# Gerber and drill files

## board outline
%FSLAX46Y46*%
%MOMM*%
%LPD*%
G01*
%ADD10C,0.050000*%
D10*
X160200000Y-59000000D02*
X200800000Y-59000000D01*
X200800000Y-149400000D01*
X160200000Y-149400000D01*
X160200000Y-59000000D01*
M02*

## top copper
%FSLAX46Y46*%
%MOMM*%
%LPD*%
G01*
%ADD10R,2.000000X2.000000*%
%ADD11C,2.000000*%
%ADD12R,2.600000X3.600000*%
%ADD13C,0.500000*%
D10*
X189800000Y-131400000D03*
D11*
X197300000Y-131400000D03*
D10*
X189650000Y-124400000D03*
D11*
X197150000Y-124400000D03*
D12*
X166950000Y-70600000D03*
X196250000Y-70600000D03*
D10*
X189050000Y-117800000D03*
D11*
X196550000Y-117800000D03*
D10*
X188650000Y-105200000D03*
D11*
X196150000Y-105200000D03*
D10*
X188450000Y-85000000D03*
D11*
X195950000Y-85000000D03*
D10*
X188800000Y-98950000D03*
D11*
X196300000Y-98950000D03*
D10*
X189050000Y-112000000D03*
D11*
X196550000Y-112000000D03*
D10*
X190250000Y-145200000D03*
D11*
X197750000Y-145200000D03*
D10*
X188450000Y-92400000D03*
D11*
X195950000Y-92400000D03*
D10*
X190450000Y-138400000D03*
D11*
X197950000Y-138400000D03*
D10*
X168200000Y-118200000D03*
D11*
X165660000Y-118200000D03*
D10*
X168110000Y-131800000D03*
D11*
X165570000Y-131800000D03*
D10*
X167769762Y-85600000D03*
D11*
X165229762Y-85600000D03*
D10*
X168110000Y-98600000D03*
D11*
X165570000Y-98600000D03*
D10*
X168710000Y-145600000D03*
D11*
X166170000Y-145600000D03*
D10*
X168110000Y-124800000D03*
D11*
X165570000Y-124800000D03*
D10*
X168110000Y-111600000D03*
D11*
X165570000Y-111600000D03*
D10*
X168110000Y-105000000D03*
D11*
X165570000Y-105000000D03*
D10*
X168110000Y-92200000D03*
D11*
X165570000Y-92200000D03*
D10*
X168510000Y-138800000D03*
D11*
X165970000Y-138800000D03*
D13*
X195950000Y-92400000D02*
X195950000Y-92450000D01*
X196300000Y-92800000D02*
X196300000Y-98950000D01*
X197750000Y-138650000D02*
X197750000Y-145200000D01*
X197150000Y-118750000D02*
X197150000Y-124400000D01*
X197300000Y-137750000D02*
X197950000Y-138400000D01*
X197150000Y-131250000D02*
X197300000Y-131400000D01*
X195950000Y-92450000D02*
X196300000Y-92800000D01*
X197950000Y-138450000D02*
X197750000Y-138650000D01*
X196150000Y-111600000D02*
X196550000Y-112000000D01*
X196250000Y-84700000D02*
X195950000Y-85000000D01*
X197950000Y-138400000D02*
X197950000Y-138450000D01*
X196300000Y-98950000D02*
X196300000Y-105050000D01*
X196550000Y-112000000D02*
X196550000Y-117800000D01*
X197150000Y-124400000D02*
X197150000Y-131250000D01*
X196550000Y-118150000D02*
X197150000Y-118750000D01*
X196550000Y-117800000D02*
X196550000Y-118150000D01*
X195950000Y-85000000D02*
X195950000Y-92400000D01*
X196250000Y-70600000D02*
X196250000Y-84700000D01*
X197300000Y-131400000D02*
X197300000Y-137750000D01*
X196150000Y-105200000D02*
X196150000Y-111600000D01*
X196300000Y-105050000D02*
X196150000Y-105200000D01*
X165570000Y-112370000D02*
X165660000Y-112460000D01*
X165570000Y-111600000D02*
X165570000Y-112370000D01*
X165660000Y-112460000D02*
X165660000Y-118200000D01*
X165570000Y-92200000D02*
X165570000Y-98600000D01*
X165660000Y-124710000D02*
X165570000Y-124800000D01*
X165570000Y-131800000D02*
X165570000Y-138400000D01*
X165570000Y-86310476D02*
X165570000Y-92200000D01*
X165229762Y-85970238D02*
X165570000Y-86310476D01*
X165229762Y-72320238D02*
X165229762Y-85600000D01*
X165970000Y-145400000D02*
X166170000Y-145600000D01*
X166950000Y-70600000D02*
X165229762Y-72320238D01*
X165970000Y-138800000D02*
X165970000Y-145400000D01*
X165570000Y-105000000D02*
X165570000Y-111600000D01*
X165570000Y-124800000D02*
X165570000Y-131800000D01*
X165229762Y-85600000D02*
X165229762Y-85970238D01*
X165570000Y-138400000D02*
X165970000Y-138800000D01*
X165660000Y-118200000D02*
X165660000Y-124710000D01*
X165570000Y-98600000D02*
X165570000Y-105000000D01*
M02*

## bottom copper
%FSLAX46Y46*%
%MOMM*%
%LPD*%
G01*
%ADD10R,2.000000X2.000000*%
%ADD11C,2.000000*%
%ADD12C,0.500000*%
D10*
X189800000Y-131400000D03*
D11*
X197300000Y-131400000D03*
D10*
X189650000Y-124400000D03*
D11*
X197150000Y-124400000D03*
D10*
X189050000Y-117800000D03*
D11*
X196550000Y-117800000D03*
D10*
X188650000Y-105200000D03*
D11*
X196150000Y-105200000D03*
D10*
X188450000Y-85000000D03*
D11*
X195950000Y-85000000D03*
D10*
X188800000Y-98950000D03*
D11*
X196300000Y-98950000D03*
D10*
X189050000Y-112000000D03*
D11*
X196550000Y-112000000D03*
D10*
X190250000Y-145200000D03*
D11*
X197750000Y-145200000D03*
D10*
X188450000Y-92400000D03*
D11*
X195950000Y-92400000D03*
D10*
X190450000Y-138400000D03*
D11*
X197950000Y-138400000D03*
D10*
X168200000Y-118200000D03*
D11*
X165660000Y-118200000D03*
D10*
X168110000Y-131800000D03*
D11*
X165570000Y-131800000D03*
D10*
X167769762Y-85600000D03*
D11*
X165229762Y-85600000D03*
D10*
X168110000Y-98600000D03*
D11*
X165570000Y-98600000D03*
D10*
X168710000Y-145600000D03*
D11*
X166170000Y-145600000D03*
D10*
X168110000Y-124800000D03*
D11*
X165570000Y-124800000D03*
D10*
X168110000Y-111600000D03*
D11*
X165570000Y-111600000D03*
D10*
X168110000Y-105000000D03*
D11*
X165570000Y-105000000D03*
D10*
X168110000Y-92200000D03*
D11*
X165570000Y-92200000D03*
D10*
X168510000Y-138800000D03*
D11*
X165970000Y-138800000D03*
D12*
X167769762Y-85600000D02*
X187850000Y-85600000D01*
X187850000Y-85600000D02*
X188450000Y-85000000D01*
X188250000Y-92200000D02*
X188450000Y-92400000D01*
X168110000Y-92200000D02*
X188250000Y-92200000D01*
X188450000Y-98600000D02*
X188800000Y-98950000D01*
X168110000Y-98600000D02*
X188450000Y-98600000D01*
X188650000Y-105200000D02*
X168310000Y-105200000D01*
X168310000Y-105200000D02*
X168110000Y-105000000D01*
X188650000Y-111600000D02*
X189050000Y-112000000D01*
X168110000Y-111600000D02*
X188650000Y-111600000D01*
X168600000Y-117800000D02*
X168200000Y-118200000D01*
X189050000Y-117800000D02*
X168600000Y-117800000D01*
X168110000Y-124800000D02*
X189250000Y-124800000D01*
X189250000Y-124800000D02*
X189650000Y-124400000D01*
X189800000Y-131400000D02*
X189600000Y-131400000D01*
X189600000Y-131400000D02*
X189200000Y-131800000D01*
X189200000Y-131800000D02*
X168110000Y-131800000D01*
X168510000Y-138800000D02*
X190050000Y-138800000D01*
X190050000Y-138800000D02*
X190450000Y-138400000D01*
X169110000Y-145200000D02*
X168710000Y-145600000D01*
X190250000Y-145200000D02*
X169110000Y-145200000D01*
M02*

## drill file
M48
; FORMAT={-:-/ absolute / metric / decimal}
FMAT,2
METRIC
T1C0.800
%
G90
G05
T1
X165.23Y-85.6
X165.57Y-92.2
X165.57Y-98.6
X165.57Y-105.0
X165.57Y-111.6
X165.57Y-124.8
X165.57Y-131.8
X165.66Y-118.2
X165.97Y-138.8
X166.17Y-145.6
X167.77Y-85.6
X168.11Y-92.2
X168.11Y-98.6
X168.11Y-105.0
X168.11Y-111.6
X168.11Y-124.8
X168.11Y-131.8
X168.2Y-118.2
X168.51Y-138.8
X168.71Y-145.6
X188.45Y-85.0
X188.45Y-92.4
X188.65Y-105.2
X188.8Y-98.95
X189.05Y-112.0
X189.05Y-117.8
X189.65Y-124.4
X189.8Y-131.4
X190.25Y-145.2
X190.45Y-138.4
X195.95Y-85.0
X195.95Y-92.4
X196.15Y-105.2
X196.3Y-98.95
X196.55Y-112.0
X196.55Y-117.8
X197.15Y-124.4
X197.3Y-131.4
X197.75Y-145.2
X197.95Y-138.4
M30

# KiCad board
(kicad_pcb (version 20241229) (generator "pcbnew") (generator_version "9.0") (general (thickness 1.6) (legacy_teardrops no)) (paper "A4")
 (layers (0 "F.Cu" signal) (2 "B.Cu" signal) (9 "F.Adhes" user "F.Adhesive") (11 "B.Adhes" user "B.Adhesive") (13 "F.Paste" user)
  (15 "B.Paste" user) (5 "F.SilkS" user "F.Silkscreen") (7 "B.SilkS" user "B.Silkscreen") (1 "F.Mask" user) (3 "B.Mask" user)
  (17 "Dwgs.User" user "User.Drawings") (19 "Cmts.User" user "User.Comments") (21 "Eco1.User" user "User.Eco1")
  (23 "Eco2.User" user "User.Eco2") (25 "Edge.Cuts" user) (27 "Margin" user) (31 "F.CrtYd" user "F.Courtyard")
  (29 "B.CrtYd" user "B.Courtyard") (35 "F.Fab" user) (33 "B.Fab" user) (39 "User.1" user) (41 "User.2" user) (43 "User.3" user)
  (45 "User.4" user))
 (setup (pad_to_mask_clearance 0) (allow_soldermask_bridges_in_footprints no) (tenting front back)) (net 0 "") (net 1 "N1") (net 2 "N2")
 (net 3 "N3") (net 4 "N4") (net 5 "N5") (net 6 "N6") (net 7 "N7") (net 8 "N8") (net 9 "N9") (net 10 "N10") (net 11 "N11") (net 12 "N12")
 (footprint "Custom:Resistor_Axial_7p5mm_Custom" (layer "F.Cu") (at 189.8 131.4)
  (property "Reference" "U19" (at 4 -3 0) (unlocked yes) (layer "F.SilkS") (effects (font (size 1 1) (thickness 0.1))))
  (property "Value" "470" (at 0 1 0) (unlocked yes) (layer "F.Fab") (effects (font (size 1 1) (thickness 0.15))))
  (pad "1" thru_hole rect (at 0 0) (size 2 2) (drill 0.8) (layers "*.Cu" "*.Mask") (remove_unused_layers no) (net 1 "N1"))
  (pad "2" thru_hole circle (at 7.5 0) (size 2 2) (drill 0.8) (layers "*.Cu" "*.Mask") (remove_unused_layers no) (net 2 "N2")))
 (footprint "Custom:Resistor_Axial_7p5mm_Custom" (layer "F.Cu") (at 189.65 124.4)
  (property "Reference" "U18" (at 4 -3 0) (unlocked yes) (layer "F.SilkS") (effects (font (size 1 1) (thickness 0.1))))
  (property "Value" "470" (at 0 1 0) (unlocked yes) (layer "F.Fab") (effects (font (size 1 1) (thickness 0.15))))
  (pad "1" thru_hole rect (at 0 0) (size 2 2) (drill 0.8) (layers "*.Cu" "*.Mask") (remove_unused_layers no) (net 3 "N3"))
  (pad "2" thru_hole circle (at 7.5 0) (size 2 2) (drill 0.8) (layers "*.Cu" "*.Mask") (remove_unused_layers no) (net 2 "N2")))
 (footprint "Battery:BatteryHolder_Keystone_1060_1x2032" (layer "F.Cu") (at 181.6 70.6)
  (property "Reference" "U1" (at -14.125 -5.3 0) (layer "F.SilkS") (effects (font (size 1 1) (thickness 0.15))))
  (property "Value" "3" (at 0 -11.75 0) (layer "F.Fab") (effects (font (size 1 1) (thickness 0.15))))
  (pad "1" smd rect (at -14.65 0 180) (size 2.6 3.6) (layers "F.Cu" "F.Mask" "F.Paste") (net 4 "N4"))
  (pad "2" smd rect (at 14.65 0 180) (size 2.6 3.6) (layers "F.Cu" "F.Mask" "F.Paste") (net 2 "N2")))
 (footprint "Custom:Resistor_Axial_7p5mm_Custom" (layer "F.Cu") (at 189.05 117.8)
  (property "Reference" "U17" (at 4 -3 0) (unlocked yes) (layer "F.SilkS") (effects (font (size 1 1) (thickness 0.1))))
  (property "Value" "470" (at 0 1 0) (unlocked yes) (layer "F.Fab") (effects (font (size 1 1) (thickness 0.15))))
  (pad "1" thru_hole rect (at 0 0) (size 2 2) (drill 0.8) (layers "*.Cu" "*.Mask") (remove_unused_layers no) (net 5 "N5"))
  (pad "2" thru_hole circle (at 7.5 0) (size 2 2) (drill 0.8) (layers "*.Cu" "*.Mask") (remove_unused_layers no) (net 2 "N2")))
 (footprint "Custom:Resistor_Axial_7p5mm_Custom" (layer "F.Cu") (at 188.65 105.2)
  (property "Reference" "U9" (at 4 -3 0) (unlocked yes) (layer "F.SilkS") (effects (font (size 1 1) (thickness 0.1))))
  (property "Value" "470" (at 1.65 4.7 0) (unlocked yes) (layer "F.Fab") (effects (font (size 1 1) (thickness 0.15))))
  (pad "1" thru_hole rect (at 0 0) (size 2 2) (drill 0.8) (layers "*.Cu" "*.Mask") (remove_unused_layers no) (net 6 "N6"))
  (pad "2" thru_hole circle (at 7.5 0) (size 2 2) (drill 0.8) (layers "*.Cu" "*.Mask") (remove_unused_layers no) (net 2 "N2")))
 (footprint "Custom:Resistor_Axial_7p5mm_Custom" (layer "F.Cu") (at 188.45 85)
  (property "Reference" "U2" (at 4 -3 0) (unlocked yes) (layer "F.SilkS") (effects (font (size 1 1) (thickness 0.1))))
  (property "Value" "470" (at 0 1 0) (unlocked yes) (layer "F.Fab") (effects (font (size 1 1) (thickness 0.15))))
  (pad "1" thru_hole rect (at 0 0) (size 2 2) (drill 0.8) (layers "*.Cu" "*.Mask") (remove_unused_layers no) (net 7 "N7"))
  (pad "2" thru_hole circle (at 7.5 0) (size 2 2) (drill 0.8) (layers "*.Cu" "*.Mask") (remove_unused_layers no) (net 2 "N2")))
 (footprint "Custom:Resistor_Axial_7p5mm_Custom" (layer "F.Cu") (at 188.8 98.95)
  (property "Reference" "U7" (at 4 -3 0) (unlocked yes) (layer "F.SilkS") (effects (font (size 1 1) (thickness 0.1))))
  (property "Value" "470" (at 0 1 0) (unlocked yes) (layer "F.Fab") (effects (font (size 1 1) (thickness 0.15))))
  (pad "1" thru_hole rect (at 0 0) (size 2 2) (drill 0.8) (layers "*.Cu" "*.Mask") (remove_unused_layers no) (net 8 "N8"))
  (pad "2" thru_hole circle (at 7.5 0) (size 2 2) (drill 0.8) (layers "*.Cu" "*.Mask") (remove_unused_layers no) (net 2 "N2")))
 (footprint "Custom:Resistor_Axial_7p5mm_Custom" (layer "F.Cu") (at 189.05 112)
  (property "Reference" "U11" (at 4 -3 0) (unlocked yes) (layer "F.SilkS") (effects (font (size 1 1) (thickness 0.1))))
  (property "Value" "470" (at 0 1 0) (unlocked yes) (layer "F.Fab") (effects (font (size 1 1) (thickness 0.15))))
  (pad "1" thru_hole rect (at 0 0) (size 2 2) (drill 0.8) (layers "*.Cu" "*.Mask") (remove_unused_layers no) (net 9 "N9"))
  (pad "2" thru_hole circle (at 7.5 0) (size 2 2) (drill 0.8) (layers "*.Cu" "*.Mask") (remove_unused_layers no) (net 2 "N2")))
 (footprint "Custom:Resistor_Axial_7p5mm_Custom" (layer "F.Cu") (at 190.25 145.2)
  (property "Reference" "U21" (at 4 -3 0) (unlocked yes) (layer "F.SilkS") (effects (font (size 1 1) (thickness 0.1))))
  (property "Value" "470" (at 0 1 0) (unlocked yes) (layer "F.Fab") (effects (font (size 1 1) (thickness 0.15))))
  (pad "1" thru_hole rect (at 0 0) (size 2 2) (drill 0.8) (layers "*.Cu" "*.Mask") (remove_unused_layers no) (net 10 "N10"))
  (pad "2" thru_hole circle (at 7.5 0) (size 2 2) (drill 0.8) (layers "*.Cu" "*.Mask") (remove_unused_layers no) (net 2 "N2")))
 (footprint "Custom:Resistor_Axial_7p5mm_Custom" (layer "F.Cu") (at 188.45 92.4)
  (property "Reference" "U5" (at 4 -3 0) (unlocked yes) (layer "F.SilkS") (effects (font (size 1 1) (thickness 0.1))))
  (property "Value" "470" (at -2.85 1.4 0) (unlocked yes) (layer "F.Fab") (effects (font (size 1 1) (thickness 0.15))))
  (pad "1" thru_hole rect (at 0 0) (size 2 2) (drill 0.8) (layers "*.Cu" "*.Mask") (remove_unused_layers no) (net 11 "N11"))
  (pad "2" thru_hole circle (at 7.5 0) (size 2 2) (drill 0.8) (layers "*.Cu" "*.Mask") (remove_unused_layers no) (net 2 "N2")))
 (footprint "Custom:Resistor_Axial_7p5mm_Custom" (layer "F.Cu") (at 190.45 138.4)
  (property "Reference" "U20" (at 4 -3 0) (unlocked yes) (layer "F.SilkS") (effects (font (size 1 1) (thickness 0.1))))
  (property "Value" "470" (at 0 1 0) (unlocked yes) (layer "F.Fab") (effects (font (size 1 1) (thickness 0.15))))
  (pad "1" thru_hole rect (at 0 0) (size 2 2) (drill 0.8) (layers "*.Cu" "*.Mask") (remove_unused_layers no) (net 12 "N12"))
  (pad "2" thru_hole circle (at 7.5 0) (size 2 2) (drill 0.8) (layers "*.Cu" "*.Mask") (remove_unused_layers no) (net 2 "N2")))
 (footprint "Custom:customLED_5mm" (layer "B.Cu") (at 168.2 118.2 180)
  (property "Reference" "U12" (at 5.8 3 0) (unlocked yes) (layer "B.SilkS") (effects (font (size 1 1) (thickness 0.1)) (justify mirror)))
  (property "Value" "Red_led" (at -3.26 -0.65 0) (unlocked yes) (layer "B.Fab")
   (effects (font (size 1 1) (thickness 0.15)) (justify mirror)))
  (pad "1" thru_hole rect (at 0 0 180) (size 2 2) (drill 0.8) (layers "*.Cu" "*.Mask") (remove_unused_layers no) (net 5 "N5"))
  (pad "2" thru_hole circle (at 2.54 0 180) (size 2 2) (drill 0.8) (layers "*.Cu" "*.Mask") (remove_unused_layers no) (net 4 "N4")))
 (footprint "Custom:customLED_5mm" (layer "B.Cu") (at 168.11 131.8 180)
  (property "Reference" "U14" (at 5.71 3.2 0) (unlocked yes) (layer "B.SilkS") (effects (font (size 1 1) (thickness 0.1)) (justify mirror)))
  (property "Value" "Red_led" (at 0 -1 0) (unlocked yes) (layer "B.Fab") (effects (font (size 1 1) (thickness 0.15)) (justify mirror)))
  (pad "1" thru_hole rect (at 0 0 180) (size 2 2) (drill 0.8) (layers "*.Cu" "*.Mask") (remove_unused_layers no) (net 1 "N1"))
  (pad "2" thru_hole circle (at 2.54 0 180) (size 2 2) (drill 0.8) (layers "*.Cu" "*.Mask") (remove_unused_layers no) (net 4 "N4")))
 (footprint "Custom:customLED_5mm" (layer "B.Cu") (at 167.769762 85.6 180)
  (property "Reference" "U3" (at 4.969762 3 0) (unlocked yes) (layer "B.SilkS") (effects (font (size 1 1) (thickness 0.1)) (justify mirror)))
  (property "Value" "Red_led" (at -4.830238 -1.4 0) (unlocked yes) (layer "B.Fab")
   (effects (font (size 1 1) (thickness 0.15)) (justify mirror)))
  (pad "1" thru_hole rect (at 0 0 180) (size 2 2) (drill 0.8) (layers "*.Cu" "*.Mask") (remove_unused_layers no) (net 7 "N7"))
  (pad "2" thru_hole circle (at 2.54 0 180) (size 2 2) (drill 0.8) (layers "*.Cu" "*.Mask") (remove_unused_layers no) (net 4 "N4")))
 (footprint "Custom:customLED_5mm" (layer "B.Cu") (at 168.11 98.6 180)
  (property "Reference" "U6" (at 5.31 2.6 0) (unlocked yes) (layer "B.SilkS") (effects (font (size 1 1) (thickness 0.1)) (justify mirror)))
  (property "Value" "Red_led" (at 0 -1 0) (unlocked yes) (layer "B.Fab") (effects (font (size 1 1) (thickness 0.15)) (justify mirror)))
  (pad "1" thru_hole rect (at 0 0 180) (size 2 2) (drill 0.8) (layers "*.Cu" "*.Mask") (remove_unused_layers no) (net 8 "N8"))
  (pad "2" thru_hole circle (at 2.54 0 180) (size 2 2) (drill 0.8) (layers "*.Cu" "*.Mask") (remove_unused_layers no) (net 4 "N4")))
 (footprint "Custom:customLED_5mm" (layer "B.Cu") (at 168.71 145.6 180)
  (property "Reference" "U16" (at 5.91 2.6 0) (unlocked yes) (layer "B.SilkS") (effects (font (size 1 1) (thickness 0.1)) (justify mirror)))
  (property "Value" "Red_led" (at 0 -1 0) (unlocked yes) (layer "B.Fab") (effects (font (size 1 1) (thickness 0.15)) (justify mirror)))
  (pad "1" thru_hole rect (at 0 0 180) (size 2 2) (drill 0.8) (layers "*.Cu" "*.Mask") (remove_unused_layers no) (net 10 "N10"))
  (pad "2" thru_hole circle (at 2.54 0 180) (size 2 2) (drill 0.8) (layers "*.Cu" "*.Mask") (remove_unused_layers no) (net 4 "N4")))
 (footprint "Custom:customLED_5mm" (layer "B.Cu") (at 168.11 124.8 180)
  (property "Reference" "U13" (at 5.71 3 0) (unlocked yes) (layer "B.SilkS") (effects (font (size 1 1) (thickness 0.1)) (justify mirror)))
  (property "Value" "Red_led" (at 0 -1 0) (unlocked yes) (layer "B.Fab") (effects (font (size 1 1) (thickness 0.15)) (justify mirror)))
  (pad "1" thru_hole rect (at 0 0 180) (size 2 2) (drill 0.8) (layers "*.Cu" "*.Mask") (remove_unused_layers no) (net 3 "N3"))
  (pad "2" thru_hole circle (at 2.54 0 180) (size 2 2) (drill 0.8) (layers "*.Cu" "*.Mask") (remove_unused_layers no) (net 4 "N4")))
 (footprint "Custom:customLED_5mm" (layer "B.Cu") (at 168.11 111.6 180)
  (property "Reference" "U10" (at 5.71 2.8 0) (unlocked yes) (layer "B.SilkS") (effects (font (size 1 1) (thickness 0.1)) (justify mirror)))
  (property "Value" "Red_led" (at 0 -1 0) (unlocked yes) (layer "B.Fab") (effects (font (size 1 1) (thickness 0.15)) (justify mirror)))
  (pad "1" thru_hole rect (at 0 0 180) (size 2 2) (drill 0.8) (layers "*.Cu" "*.Mask") (remove_unused_layers no) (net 9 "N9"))
  (pad "2" thru_hole circle (at 2.54 0 180) (size 2 2) (drill 0.8) (layers "*.Cu" "*.Mask") (remove_unused_layers no) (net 4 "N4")))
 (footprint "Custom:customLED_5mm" (layer "B.Cu") (at 168.11 105 180)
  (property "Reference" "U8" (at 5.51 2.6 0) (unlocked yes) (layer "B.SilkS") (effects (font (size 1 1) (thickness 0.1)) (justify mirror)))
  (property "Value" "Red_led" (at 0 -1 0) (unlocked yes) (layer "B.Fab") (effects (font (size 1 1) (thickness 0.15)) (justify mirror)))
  (pad "1" thru_hole rect (at 0 0 180) (size 2 2) (drill 0.8) (layers "*.Cu" "*.Mask") (remove_unused_layers no) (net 6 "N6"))
  (pad "2" thru_hole circle (at 2.54 0 180) (size 2 2) (drill 0.8) (layers "*.Cu" "*.Mask") (remove_unused_layers no) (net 4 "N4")))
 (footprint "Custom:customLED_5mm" (layer "B.Cu") (at 168.11 92.2 180)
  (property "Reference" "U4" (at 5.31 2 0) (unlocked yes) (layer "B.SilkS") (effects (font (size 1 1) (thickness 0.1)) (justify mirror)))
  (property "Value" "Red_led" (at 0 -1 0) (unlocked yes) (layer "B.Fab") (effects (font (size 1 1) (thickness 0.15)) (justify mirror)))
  (pad "1" thru_hole rect (at 0 0 180) (size 2 2) (drill 0.8) (layers "*.Cu" "*.Mask") (remove_unused_layers no) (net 11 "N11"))
  (pad "2" thru_hole circle (at 2.54 0 180) (size 2 2) (drill 0.8) (layers "*.Cu" "*.Mask") (remove_unused_layers no) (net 4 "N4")))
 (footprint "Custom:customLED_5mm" (layer "B.Cu") (at 168.51 138.8 180)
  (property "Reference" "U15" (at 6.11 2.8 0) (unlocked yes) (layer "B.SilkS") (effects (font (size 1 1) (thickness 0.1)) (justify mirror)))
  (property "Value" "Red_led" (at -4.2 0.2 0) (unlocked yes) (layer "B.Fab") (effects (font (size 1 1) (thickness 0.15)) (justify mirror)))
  (pad "1" thru_hole rect (at 0 0 180) (size 2 2) (drill 0.8) (layers "*.Cu" "*.Mask") (remove_unused_layers no) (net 12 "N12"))
  (pad "2" thru_hole circle (at 2.54 0 180) (size 2 2) (drill 0.8) (layers "*.Cu" "*.Mask") (remove_unused_layers no) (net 4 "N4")))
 (gr_rect (start 160.2 59) (end 200.8 149.4) (stroke (width 0.05) (type default)) (fill no) (layer "Edge.Cuts"))
 (segment (start 195.95 92.4) (end 195.95 92.45) (width 0.5) (layer "F.Cu") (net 2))
 (segment (start 196.3 92.8) (end 196.3 98.95) (width 0.5) (layer "F.Cu") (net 2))
 (segment (start 197.75 138.65) (end 197.75 145.2) (width 0.5) (layer "F.Cu") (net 2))
 (segment (start 197.15 118.75) (end 197.15 124.4) (width 0.5) (layer "F.Cu") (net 2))
 (segment (start 197.3 137.75) (end 197.95 138.4) (width 0.5) (layer "F.Cu") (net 2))
 (segment (start 197.15 131.25) (end 197.3 131.4) (width 0.5) (layer "F.Cu") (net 2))
 (segment (start 195.95 92.45) (end 196.3 92.8) (width 0.5) (layer "F.Cu") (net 2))
 (segment (start 197.95 138.45) (end 197.75 138.65) (width 0.5) (layer "F.Cu") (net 2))
 (segment (start 196.15 111.6) (end 196.55 112) (width 0.5) (layer "F.Cu") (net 2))
 (segment (start 196.25 84.7) (end 195.95 85) (width 0.5) (layer "F.Cu") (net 2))
 (segment (start 197.95 138.4) (end 197.95 138.45) (width 0.5) (layer "F.Cu") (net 2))
 (segment (start 196.3 98.95) (end 196.3 105.05) (width 0.5) (layer "F.Cu") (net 2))
 (segment (start 196.55 112) (end 196.55 117.8) (width 0.5) (layer "F.Cu") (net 2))
 (segment (start 197.15 124.4) (end 197.15 131.25) (width 0.5) (layer "F.Cu") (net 2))
 (segment (start 196.55 118.15) (end 197.15 118.75) (width 0.5) (layer "F.Cu") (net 2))
 (segment (start 196.55 117.8) (end 196.55 118.15) (width 0.5) (layer "F.Cu") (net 2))
 (segment (start 195.95 85) (end 195.95 92.4) (width 0.5) (layer "F.Cu") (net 2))
 (segment (start 196.25 70.6) (end 196.25 84.7) (width 0.5) (layer "F.Cu") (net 2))
 (segment (start 197.3 131.4) (end 197.3 137.75) (width 0.5) (layer "F.Cu") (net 2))
 (segment (start 196.15 105.2) (end 196.15 111.6) (width 0.5) (layer "F.Cu") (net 2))
 (segment (start 196.3 105.05) (end 196.15 105.2) (width 0.5) (layer "F.Cu") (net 2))
 (segment (start 165.57 112.37) (end 165.66 112.46) (width 0.5) (layer "F.Cu") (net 4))
 (segment (start 165.57 111.6) (end 165.57 112.37) (width 0.5) (layer "F.Cu") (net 4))
 (segment (start 165.66 112.46) (end 165.66 118.2) (width 0.5) (layer "F.Cu") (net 4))
 (segment (start 165.57 92.2) (end 165.57 98.6) (width 0.5) (layer "F.Cu") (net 4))
 (segment (start 165.66 124.71) (end 165.57 124.8) (width 0.5) (layer "F.Cu") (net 4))
 (segment (start 165.57 131.8) (end 165.57 138.4) (width 0.5) (layer "F.Cu") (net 4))
 (segment (start 165.57 86.310476) (end 165.57 92.2) (width 0.5) (layer "F.Cu") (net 4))
 (segment (start 165.229762 85.970238) (end 165.57 86.310476) (width 0.5) (layer "F.Cu") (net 4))
 (segment (start 165.229762 72.320238) (end 165.229762 85.6) (width 0.5) (layer "F.Cu") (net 4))
 (segment (start 165.97 145.4) (end 166.17 145.6) (width 0.5) (layer "F.Cu") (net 4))
 (segment (start 166.95 70.6) (end 165.229762 72.320238) (width 0.5) (layer "F.Cu") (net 4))
 (segment (start 165.97 138.8) (end 165.97 145.4) (width 0.5) (layer "F.Cu") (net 4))
 (segment (start 165.57 105) (end 165.57 111.6) (width 0.5) (layer "F.Cu") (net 4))
 (segment (start 165.57 124.8) (end 165.57 131.8) (width 0.5) (layer "F.Cu") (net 4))
 (segment (start 165.229762 85.6) (end 165.229762 85.970238) (width 0.5) (layer "F.Cu") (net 4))
 (segment (start 165.57 138.4) (end 165.97 138.8) (width 0.5) (layer "F.Cu") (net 4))
 (segment (start 165.66 118.2) (end 165.66 124.71) (width 0.5) (layer "F.Cu") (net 4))
 (segment (start 165.57 98.6) (end 165.57 105) (width 0.5) (layer "F.Cu") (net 4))
 (segment (start 167.769762 85.6) (end 187.85 85.6) (width 0.5) (layer "B.Cu") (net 7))
 (segment (start 187.85 85.6) (end 188.45 85) (width 0.5) (layer "B.Cu") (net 7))
 (segment (start 188.25 92.2) (end 188.45 92.4) (width 0.5) (layer "B.Cu") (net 11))
 (segment (start 168.11 92.2) (end 188.25 92.2) (width 0.5) (layer "B.Cu") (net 11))
 (segment (start 188.45 98.6) (end 188.8 98.95) (width 0.5) (layer "B.Cu") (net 8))
 (segment (start 168.11 98.6) (end 188.45 98.6) (width 0.5) (layer "B.Cu") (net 8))
 (segment (start 188.65 105.2) (end 168.31 105.2) (width 0.5) (layer "B.Cu") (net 6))
 (segment (start 168.31 105.2) (end 168.11 105) (width 0.5) (layer "B.Cu") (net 6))
 (segment (start 188.65 111.6) (end 189.05 112) (width 0.5) (layer "B.Cu") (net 9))
 (segment (start 168.11 111.6) (end 188.65 111.6) (width 0.5) (layer "B.Cu") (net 9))
 (segment (start 168.6 117.8) (end 168.2 118.2) (width 0.5) (layer "B.Cu") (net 5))
 (segment (start 189.05 117.8) (end 168.6 117.8) (width 0.5) (layer "B.Cu") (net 5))
 (segment (start 168.11 124.8) (end 189.25 124.8) (width 0.5) (layer "B.Cu") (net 3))
 (segment (start 189.25 124.8) (end 189.65 124.4) (width 0.5) (layer "B.Cu") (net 3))
 (segment (start 189.8 131.4) (end 189.6 131.4) (width 0.5) (layer "B.Cu") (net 1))
 (segment (start 189.6 131.4) (end 189.2 131.8) (width 0.5) (layer "B.Cu") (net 1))
 (segment (start 189.2 131.8) (end 168.11 131.8) (width 0.5) (layer "B.Cu") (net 1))
 (segment (start 168.51 138.8) (end 190.05 138.8) (width 0.5) (layer "B.Cu") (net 12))
 (segment (start 190.05 138.8) (end 190.45 138.4) (width 0.5) (layer "B.Cu") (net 12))
 (segment (start 169.11 145.2) (end 168.71 145.6) (width 0.5) (layer "B.Cu") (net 10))
 (segment (start 190.25 145.2) (end 169.11 145.2) (width 0.5) (layer "B.Cu") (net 10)))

